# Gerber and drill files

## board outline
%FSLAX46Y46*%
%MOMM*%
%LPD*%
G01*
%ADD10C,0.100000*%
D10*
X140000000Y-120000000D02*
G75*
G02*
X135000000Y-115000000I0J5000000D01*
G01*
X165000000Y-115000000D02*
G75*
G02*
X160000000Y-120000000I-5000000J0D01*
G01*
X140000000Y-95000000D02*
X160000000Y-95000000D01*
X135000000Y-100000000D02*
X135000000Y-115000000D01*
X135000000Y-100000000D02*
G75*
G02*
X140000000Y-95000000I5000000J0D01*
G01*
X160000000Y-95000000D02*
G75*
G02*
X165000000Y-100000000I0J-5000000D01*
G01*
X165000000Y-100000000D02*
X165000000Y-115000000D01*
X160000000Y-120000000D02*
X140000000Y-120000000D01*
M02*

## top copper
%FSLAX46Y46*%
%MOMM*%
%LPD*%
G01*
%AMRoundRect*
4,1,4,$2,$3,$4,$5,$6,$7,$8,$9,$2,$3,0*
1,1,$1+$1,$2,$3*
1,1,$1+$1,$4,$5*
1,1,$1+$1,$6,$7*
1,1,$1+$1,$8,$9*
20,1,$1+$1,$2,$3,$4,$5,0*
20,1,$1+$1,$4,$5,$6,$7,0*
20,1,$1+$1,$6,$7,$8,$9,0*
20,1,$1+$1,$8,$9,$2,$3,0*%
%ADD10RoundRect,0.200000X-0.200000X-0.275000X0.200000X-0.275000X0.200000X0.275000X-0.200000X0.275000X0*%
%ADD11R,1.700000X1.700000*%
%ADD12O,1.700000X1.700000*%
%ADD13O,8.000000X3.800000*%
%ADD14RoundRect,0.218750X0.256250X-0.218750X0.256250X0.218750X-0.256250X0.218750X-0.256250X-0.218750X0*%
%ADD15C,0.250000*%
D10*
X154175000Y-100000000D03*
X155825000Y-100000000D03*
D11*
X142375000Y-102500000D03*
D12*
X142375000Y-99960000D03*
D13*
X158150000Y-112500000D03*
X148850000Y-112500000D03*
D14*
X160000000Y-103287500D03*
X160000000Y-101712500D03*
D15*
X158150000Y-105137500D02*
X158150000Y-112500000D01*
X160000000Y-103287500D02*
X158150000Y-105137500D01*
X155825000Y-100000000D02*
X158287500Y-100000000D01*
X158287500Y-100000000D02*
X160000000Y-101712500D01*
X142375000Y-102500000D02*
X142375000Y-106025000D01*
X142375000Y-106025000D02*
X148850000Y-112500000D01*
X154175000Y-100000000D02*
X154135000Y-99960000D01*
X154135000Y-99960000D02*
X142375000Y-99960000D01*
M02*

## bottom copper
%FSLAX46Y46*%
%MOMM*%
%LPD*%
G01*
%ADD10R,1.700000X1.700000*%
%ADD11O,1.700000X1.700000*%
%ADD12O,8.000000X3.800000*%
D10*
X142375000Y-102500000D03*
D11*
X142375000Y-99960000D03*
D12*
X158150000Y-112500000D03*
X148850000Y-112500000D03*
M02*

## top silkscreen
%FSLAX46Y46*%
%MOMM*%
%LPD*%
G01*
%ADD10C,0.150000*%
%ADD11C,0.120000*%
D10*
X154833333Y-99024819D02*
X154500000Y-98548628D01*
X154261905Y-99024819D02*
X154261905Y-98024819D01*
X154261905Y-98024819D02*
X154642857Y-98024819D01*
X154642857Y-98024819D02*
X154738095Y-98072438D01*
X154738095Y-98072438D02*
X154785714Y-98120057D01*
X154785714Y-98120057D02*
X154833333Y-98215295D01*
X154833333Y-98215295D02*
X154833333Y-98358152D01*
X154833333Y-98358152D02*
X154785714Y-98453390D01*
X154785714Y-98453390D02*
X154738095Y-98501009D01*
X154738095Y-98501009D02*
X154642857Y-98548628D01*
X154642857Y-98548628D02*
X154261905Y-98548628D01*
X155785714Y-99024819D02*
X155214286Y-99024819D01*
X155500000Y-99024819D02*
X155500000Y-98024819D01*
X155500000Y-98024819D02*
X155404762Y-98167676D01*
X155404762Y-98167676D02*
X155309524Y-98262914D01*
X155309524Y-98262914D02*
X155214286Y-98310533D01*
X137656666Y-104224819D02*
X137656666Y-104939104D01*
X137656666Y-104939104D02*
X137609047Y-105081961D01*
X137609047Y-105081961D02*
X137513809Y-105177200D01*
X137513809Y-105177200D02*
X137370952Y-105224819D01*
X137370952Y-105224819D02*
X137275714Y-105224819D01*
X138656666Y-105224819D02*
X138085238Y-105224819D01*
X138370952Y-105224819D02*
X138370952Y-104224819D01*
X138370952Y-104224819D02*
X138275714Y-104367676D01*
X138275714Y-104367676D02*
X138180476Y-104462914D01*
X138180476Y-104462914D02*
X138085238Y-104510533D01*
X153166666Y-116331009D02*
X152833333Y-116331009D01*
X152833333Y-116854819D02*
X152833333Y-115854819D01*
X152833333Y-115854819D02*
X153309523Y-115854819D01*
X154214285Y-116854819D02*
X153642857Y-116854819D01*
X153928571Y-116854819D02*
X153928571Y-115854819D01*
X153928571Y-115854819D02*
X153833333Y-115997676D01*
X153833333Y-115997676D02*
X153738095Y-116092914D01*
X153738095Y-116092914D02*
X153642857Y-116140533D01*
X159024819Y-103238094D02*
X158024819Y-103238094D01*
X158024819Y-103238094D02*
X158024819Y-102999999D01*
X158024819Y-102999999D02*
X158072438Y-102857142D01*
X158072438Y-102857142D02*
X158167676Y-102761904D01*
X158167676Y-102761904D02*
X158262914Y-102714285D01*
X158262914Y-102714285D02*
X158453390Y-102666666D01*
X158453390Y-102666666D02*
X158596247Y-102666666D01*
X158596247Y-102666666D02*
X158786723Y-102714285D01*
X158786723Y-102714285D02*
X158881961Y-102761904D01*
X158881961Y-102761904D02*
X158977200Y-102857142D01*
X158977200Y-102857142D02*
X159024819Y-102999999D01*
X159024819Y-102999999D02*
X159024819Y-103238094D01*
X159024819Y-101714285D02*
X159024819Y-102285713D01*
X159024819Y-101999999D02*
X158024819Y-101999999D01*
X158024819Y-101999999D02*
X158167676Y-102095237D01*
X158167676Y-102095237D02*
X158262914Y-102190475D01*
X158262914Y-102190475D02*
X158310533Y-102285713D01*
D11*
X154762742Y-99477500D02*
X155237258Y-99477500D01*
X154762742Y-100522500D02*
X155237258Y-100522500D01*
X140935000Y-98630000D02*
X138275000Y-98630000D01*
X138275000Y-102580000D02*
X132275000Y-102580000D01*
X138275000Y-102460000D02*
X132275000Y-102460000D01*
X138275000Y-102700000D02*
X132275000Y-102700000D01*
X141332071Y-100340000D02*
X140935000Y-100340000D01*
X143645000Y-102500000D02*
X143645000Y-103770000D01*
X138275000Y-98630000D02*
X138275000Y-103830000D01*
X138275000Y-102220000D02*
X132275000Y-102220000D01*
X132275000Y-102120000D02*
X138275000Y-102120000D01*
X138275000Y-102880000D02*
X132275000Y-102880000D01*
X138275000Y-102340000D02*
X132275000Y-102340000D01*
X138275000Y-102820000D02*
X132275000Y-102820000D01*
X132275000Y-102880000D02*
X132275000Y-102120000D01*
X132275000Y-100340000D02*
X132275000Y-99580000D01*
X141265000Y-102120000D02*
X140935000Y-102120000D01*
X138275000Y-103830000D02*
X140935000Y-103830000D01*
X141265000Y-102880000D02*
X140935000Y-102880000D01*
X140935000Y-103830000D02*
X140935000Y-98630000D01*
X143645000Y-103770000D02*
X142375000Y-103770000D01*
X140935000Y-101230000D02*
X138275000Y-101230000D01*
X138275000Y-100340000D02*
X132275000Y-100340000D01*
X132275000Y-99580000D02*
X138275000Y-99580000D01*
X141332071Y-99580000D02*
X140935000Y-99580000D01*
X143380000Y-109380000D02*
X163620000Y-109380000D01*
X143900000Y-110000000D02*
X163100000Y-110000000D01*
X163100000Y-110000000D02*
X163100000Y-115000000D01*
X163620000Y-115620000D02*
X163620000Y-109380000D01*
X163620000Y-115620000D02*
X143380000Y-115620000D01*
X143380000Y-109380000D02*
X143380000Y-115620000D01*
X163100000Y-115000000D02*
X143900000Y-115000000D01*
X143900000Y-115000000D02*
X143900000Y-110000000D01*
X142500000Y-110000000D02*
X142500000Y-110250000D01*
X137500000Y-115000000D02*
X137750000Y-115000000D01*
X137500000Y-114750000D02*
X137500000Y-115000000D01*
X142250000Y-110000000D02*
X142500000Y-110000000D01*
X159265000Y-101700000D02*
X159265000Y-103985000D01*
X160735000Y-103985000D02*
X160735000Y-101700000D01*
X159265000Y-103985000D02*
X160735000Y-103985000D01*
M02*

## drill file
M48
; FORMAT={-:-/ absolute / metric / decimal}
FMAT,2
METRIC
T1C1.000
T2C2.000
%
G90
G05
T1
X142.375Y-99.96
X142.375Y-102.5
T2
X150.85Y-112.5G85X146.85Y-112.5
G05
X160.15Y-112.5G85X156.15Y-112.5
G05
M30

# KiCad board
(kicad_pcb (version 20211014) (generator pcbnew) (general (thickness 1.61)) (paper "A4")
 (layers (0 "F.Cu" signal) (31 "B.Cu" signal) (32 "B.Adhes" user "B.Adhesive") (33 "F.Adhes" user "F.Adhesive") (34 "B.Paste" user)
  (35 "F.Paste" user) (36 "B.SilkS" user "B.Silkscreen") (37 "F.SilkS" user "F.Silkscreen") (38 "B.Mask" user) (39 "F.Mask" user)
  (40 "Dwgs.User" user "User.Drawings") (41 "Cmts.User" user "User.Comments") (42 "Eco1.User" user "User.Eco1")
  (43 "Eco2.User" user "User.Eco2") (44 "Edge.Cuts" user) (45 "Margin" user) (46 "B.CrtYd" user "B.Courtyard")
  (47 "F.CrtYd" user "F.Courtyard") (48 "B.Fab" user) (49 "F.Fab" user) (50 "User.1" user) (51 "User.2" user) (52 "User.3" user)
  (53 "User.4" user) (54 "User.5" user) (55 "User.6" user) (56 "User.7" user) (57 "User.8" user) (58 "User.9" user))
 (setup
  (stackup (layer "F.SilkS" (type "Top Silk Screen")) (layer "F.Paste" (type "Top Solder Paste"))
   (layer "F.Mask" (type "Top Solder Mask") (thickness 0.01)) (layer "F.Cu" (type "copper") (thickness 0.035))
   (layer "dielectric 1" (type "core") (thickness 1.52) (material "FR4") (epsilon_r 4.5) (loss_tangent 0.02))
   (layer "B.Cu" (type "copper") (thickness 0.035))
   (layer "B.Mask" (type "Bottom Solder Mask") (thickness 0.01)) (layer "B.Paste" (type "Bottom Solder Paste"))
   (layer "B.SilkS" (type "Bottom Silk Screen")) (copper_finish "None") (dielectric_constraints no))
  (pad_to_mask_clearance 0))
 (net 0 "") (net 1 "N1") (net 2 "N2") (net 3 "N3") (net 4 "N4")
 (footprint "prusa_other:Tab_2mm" (layer "F.Cu") (at 155 95 -90)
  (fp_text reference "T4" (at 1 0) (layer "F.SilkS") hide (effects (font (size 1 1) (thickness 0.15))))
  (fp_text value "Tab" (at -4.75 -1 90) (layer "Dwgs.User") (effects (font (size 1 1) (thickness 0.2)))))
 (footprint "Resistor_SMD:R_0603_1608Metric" (layer "F.Cu") (at 155 100)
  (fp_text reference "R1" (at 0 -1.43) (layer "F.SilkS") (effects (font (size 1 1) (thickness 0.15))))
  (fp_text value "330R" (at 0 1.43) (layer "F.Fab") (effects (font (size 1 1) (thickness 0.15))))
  (fp_line (start -0.237258 -0.5225) (end 0.237258 -0.5225) (layer "F.SilkS") (width 0.12))
  (fp_line (start -0.237258 0.5225) (end 0.237258 0.5225) (layer "F.SilkS") (width 0.12))
  (pad "1" smd roundrect (at -0.825 0) (size 0.8 0.95) (layers "F.Cu" "F.Paste" "F.Mask") (roundrect_rratio 0.25) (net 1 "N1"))
  (pad "2" smd roundrect (at 0.825 0) (size 0.8 0.95) (layers "F.Cu" "F.Paste" "F.Mask") (roundrect_rratio 0.25) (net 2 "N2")))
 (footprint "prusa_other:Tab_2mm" (layer "F.Cu") (at 135 110)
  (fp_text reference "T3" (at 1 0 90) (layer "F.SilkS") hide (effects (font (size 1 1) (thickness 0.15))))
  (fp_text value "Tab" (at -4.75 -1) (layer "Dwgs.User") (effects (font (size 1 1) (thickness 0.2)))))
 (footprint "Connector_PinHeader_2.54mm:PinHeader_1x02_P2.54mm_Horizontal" (layer "F.Cu") (at 142.375 102.5 180)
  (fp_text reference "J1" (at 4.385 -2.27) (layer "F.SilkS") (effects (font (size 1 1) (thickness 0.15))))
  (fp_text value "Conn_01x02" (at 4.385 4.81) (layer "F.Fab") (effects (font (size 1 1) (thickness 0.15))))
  (fp_line (start 1.44 3.87) (end 4.1 3.87) (layer "F.SilkS") (width 0.12))
  (fp_line (start 4.1 -0.08) (end 10.1 -0.08) (layer "F.SilkS") (width 0.12))
  (fp_line (start 4.1 0.04) (end 10.1 0.04) (layer "F.SilkS") (width 0.12))
  (fp_line (start 4.1 -0.2) (end 10.1 -0.2) (layer "F.SilkS") (width 0.12))
  (fp_line (start 1.042929 2.16) (end 1.44 2.16) (layer "F.SilkS") (width 0.12))
  (fp_line (start -1.27 0) (end -1.27 -1.27) (layer "F.SilkS") (width 0.12))
  (fp_line (start 4.1 3.87) (end 4.1 -1.33) (layer "F.SilkS") (width 0.12))
  (fp_line (start 4.1 0.28) (end 10.1 0.28) (layer "F.SilkS") (width 0.12))
  (fp_line (start 10.1 0.38) (end 4.1 0.38) (layer "F.SilkS") (width 0.12))
  (fp_line (start 4.1 -0.38) (end 10.1 -0.38) (layer "F.SilkS") (width 0.12))
  (fp_line (start 4.1 0.16) (end 10.1 0.16) (layer "F.SilkS") (width 0.12))
  (fp_line (start 4.1 -0.32) (end 10.1 -0.32) (layer "F.SilkS") (width 0.12))
  (fp_line (start 10.1 -0.38) (end 10.1 0.38) (layer "F.SilkS") (width 0.12))
  (fp_line (start 10.1 2.16) (end 10.1 2.92) (layer "F.SilkS") (width 0.12))
  (fp_line (start 1.11 0.38) (end 1.44 0.38) (layer "F.SilkS") (width 0.12))
  (fp_line (start 4.1 -1.33) (end 1.44 -1.33) (layer "F.SilkS") (width 0.12))
  (fp_line (start 1.11 -0.38) (end 1.44 -0.38) (layer "F.SilkS") (width 0.12))
  (fp_line (start 1.44 -1.33) (end 1.44 3.87) (layer "F.SilkS") (width 0.12))
  (fp_line (start -1.27 -1.27) (end 0 -1.27) (layer "F.SilkS") (width 0.12))
  (fp_line (start 1.44 1.27) (end 4.1 1.27) (layer "F.SilkS") (width 0.12))
  (fp_line (start 4.1 2.16) (end 10.1 2.16) (layer "F.SilkS") (width 0.12))
  (fp_line (start 10.1 2.92) (end 4.1 2.92) (layer "F.SilkS") (width 0.12))
  (fp_line (start 1.042929 2.92) (end 1.44 2.92) (layer "F.SilkS") (width 0.12))
  (pad "1" thru_hole rect (at 0 0 180) (size 1.7 1.7) (drill 1) (layers *.Cu *.Mask) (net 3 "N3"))
  (pad "2" thru_hole oval (at 0 2.54 180) (size 1.7 1.7) (drill 1) (layers *.Cu *.Mask) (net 1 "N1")))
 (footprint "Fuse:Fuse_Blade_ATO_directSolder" (layer "F.Cu") (at 158.15 112.5 180)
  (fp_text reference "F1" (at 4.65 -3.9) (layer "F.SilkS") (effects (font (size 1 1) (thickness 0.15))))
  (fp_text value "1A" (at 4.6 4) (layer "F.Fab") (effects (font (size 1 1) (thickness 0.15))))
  (fp_line (start 14.77 3.12) (end -5.47 3.12) (layer "F.SilkS") (width 0.12))
  (fp_line (start 14.25 2.5) (end -4.95 2.5) (layer "F.SilkS") (width 0.12))
  (fp_line (start -4.95 2.5) (end -4.95 -2.5) (layer "F.SilkS") (width 0.12))
  (fp_line (start -5.47 -3.12) (end -5.47 3.12) (layer "F.SilkS") (width 0.12))
  (fp_line (start -5.47 -3.12) (end 14.77 -3.12) (layer "F.SilkS") (width 0.12))
  (fp_line (start 14.77 3.12) (end 14.77 -3.12) (layer "F.SilkS") (width 0.12))
  (fp_line (start -4.95 -2.5) (end 14.25 -2.5) (layer "F.SilkS") (width 0.12))
  (fp_line (start 14.25 -2.5) (end 14.25 2.5) (layer "F.SilkS") (width 0.12))
  (pad "1" thru_hole oval (at 0 0 180) (size 8 3.8) (drill oval 6 2) (layers *.Cu *.Mask) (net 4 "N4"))
  (pad "2" thru_hole oval (at 9.3 0 180) (size 8 3.8) (drill oval 6 2) (layers *.Cu *.Mask) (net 3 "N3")))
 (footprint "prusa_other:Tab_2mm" (layer "F.Cu") (at 155 120 90)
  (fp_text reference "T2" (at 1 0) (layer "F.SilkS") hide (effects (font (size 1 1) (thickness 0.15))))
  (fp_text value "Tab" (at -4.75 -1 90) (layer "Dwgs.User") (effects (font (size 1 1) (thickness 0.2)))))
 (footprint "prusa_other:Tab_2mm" (layer "F.Cu") (at 165 110 180)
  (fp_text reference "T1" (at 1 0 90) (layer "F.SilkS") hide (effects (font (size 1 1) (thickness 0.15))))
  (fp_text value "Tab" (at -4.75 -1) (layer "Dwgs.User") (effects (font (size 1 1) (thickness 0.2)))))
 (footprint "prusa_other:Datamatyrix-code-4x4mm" (layer "F.Cu") (at 140 112.5)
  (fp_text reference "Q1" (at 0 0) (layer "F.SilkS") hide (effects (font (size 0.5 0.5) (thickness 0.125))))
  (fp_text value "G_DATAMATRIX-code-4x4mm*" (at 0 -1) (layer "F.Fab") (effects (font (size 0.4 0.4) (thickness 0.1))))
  (fp_line (start 2.5 -2.5) (end 2.5 -2.25) (layer "F.SilkS") (width 0.12))
  (fp_line (start -2.5 2.5) (end -2.25 2.5) (layer "F.SilkS") (width 0.12))
  (fp_line (start -2.5 2.25) (end -2.5 2.5) (layer "F.SilkS") (width 0.12))
  (fp_line (start 2.25 -2.5) (end 2.5 -2.5) (layer "F.SilkS") (width 0.12)))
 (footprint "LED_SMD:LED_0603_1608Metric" (layer "F.Cu") (at 160 102.5 90)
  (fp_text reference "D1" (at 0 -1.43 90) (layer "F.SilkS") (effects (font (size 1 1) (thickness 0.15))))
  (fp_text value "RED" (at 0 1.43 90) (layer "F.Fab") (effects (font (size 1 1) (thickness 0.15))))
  (fp_line (start 0.8 -0.735) (end -1.485 -0.735) (layer "F.SilkS") (width 0.12))
  (fp_line (start -1.485 0.735) (end 0.8 0.735) (layer "F.SilkS") (width 0.12))
  (fp_line (start -1.485 -0.735) (end -1.485 0.735) (layer "F.SilkS") (width 0.12))
  (pad "1" smd roundrect (at -0.7875 0 90) (size 0.875 0.95) (layers "F.Cu" "F.Paste" "F.Mask") (roundrect_rratio 0.25) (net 4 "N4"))
  (pad "2" smd roundrect (at 0.7875 0 90) (size 0.875 0.95) (layers "F.Cu" "F.Paste" "F.Mask") (roundrect_rratio 0.25) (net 2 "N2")))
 (gr_arc (start 140 120) (mid 136.464466 118.535534) (end 135 115) (layer "Edge.Cuts") (width 0.1))
 (gr_arc (start 165 115) (mid 163.535534 118.535534) (end 160 120) (layer "Edge.Cuts") (width 0.1))
 (gr_line (start 140 95) (end 160 95) (layer "Edge.Cuts") (width 0.1))
 (gr_line (start 135 100) (end 135 115) (layer "Edge.Cuts") (width 0.1))
 (gr_arc (start 135 100) (mid 136.464466 96.464466) (end 140 95) (layer "Edge.Cuts") (width 0.1))
 (gr_arc (start 160 95) (mid 163.535534 96.464466) (end 165 100) (layer "Edge.Cuts") (width 0.1))
 (gr_line (start 165 100) (end 165 115) (layer "Edge.Cuts") (width 0.1))
 (gr_line (start 160 120) (end 140 120) (layer "Edge.Cuts") (width 0.1))
 (segment (start 158.15 105.1375) (end 158.15 112.5) (width 0.25) (layer "F.Cu") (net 4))
 (segment (start 160 103.2875) (end 158.15 105.1375) (width 0.25) (layer "F.Cu") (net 4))
 (segment (start 155.825 100) (end 158.2875 100) (width 0.25) (layer "F.Cu") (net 2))
 (segment (start 158.2875 100) (end 160 101.7125) (width 0.25) (layer "F.Cu") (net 2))
 (segment (start 142.375 102.5) (end 142.375 106.025) (width 0.25) (layer "F.Cu") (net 3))
 (segment (start 142.375 106.025) (end 148.85 112.5) (width 0.25) (layer "F.Cu") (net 3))
 (segment (start 154.175 100) (end 154.135 99.96) (width 0.25) (layer "F.Cu") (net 1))
 (segment (start 154.135 99.96) (end 142.375 99.96) (width 0.25) (layer "F.Cu") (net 1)))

